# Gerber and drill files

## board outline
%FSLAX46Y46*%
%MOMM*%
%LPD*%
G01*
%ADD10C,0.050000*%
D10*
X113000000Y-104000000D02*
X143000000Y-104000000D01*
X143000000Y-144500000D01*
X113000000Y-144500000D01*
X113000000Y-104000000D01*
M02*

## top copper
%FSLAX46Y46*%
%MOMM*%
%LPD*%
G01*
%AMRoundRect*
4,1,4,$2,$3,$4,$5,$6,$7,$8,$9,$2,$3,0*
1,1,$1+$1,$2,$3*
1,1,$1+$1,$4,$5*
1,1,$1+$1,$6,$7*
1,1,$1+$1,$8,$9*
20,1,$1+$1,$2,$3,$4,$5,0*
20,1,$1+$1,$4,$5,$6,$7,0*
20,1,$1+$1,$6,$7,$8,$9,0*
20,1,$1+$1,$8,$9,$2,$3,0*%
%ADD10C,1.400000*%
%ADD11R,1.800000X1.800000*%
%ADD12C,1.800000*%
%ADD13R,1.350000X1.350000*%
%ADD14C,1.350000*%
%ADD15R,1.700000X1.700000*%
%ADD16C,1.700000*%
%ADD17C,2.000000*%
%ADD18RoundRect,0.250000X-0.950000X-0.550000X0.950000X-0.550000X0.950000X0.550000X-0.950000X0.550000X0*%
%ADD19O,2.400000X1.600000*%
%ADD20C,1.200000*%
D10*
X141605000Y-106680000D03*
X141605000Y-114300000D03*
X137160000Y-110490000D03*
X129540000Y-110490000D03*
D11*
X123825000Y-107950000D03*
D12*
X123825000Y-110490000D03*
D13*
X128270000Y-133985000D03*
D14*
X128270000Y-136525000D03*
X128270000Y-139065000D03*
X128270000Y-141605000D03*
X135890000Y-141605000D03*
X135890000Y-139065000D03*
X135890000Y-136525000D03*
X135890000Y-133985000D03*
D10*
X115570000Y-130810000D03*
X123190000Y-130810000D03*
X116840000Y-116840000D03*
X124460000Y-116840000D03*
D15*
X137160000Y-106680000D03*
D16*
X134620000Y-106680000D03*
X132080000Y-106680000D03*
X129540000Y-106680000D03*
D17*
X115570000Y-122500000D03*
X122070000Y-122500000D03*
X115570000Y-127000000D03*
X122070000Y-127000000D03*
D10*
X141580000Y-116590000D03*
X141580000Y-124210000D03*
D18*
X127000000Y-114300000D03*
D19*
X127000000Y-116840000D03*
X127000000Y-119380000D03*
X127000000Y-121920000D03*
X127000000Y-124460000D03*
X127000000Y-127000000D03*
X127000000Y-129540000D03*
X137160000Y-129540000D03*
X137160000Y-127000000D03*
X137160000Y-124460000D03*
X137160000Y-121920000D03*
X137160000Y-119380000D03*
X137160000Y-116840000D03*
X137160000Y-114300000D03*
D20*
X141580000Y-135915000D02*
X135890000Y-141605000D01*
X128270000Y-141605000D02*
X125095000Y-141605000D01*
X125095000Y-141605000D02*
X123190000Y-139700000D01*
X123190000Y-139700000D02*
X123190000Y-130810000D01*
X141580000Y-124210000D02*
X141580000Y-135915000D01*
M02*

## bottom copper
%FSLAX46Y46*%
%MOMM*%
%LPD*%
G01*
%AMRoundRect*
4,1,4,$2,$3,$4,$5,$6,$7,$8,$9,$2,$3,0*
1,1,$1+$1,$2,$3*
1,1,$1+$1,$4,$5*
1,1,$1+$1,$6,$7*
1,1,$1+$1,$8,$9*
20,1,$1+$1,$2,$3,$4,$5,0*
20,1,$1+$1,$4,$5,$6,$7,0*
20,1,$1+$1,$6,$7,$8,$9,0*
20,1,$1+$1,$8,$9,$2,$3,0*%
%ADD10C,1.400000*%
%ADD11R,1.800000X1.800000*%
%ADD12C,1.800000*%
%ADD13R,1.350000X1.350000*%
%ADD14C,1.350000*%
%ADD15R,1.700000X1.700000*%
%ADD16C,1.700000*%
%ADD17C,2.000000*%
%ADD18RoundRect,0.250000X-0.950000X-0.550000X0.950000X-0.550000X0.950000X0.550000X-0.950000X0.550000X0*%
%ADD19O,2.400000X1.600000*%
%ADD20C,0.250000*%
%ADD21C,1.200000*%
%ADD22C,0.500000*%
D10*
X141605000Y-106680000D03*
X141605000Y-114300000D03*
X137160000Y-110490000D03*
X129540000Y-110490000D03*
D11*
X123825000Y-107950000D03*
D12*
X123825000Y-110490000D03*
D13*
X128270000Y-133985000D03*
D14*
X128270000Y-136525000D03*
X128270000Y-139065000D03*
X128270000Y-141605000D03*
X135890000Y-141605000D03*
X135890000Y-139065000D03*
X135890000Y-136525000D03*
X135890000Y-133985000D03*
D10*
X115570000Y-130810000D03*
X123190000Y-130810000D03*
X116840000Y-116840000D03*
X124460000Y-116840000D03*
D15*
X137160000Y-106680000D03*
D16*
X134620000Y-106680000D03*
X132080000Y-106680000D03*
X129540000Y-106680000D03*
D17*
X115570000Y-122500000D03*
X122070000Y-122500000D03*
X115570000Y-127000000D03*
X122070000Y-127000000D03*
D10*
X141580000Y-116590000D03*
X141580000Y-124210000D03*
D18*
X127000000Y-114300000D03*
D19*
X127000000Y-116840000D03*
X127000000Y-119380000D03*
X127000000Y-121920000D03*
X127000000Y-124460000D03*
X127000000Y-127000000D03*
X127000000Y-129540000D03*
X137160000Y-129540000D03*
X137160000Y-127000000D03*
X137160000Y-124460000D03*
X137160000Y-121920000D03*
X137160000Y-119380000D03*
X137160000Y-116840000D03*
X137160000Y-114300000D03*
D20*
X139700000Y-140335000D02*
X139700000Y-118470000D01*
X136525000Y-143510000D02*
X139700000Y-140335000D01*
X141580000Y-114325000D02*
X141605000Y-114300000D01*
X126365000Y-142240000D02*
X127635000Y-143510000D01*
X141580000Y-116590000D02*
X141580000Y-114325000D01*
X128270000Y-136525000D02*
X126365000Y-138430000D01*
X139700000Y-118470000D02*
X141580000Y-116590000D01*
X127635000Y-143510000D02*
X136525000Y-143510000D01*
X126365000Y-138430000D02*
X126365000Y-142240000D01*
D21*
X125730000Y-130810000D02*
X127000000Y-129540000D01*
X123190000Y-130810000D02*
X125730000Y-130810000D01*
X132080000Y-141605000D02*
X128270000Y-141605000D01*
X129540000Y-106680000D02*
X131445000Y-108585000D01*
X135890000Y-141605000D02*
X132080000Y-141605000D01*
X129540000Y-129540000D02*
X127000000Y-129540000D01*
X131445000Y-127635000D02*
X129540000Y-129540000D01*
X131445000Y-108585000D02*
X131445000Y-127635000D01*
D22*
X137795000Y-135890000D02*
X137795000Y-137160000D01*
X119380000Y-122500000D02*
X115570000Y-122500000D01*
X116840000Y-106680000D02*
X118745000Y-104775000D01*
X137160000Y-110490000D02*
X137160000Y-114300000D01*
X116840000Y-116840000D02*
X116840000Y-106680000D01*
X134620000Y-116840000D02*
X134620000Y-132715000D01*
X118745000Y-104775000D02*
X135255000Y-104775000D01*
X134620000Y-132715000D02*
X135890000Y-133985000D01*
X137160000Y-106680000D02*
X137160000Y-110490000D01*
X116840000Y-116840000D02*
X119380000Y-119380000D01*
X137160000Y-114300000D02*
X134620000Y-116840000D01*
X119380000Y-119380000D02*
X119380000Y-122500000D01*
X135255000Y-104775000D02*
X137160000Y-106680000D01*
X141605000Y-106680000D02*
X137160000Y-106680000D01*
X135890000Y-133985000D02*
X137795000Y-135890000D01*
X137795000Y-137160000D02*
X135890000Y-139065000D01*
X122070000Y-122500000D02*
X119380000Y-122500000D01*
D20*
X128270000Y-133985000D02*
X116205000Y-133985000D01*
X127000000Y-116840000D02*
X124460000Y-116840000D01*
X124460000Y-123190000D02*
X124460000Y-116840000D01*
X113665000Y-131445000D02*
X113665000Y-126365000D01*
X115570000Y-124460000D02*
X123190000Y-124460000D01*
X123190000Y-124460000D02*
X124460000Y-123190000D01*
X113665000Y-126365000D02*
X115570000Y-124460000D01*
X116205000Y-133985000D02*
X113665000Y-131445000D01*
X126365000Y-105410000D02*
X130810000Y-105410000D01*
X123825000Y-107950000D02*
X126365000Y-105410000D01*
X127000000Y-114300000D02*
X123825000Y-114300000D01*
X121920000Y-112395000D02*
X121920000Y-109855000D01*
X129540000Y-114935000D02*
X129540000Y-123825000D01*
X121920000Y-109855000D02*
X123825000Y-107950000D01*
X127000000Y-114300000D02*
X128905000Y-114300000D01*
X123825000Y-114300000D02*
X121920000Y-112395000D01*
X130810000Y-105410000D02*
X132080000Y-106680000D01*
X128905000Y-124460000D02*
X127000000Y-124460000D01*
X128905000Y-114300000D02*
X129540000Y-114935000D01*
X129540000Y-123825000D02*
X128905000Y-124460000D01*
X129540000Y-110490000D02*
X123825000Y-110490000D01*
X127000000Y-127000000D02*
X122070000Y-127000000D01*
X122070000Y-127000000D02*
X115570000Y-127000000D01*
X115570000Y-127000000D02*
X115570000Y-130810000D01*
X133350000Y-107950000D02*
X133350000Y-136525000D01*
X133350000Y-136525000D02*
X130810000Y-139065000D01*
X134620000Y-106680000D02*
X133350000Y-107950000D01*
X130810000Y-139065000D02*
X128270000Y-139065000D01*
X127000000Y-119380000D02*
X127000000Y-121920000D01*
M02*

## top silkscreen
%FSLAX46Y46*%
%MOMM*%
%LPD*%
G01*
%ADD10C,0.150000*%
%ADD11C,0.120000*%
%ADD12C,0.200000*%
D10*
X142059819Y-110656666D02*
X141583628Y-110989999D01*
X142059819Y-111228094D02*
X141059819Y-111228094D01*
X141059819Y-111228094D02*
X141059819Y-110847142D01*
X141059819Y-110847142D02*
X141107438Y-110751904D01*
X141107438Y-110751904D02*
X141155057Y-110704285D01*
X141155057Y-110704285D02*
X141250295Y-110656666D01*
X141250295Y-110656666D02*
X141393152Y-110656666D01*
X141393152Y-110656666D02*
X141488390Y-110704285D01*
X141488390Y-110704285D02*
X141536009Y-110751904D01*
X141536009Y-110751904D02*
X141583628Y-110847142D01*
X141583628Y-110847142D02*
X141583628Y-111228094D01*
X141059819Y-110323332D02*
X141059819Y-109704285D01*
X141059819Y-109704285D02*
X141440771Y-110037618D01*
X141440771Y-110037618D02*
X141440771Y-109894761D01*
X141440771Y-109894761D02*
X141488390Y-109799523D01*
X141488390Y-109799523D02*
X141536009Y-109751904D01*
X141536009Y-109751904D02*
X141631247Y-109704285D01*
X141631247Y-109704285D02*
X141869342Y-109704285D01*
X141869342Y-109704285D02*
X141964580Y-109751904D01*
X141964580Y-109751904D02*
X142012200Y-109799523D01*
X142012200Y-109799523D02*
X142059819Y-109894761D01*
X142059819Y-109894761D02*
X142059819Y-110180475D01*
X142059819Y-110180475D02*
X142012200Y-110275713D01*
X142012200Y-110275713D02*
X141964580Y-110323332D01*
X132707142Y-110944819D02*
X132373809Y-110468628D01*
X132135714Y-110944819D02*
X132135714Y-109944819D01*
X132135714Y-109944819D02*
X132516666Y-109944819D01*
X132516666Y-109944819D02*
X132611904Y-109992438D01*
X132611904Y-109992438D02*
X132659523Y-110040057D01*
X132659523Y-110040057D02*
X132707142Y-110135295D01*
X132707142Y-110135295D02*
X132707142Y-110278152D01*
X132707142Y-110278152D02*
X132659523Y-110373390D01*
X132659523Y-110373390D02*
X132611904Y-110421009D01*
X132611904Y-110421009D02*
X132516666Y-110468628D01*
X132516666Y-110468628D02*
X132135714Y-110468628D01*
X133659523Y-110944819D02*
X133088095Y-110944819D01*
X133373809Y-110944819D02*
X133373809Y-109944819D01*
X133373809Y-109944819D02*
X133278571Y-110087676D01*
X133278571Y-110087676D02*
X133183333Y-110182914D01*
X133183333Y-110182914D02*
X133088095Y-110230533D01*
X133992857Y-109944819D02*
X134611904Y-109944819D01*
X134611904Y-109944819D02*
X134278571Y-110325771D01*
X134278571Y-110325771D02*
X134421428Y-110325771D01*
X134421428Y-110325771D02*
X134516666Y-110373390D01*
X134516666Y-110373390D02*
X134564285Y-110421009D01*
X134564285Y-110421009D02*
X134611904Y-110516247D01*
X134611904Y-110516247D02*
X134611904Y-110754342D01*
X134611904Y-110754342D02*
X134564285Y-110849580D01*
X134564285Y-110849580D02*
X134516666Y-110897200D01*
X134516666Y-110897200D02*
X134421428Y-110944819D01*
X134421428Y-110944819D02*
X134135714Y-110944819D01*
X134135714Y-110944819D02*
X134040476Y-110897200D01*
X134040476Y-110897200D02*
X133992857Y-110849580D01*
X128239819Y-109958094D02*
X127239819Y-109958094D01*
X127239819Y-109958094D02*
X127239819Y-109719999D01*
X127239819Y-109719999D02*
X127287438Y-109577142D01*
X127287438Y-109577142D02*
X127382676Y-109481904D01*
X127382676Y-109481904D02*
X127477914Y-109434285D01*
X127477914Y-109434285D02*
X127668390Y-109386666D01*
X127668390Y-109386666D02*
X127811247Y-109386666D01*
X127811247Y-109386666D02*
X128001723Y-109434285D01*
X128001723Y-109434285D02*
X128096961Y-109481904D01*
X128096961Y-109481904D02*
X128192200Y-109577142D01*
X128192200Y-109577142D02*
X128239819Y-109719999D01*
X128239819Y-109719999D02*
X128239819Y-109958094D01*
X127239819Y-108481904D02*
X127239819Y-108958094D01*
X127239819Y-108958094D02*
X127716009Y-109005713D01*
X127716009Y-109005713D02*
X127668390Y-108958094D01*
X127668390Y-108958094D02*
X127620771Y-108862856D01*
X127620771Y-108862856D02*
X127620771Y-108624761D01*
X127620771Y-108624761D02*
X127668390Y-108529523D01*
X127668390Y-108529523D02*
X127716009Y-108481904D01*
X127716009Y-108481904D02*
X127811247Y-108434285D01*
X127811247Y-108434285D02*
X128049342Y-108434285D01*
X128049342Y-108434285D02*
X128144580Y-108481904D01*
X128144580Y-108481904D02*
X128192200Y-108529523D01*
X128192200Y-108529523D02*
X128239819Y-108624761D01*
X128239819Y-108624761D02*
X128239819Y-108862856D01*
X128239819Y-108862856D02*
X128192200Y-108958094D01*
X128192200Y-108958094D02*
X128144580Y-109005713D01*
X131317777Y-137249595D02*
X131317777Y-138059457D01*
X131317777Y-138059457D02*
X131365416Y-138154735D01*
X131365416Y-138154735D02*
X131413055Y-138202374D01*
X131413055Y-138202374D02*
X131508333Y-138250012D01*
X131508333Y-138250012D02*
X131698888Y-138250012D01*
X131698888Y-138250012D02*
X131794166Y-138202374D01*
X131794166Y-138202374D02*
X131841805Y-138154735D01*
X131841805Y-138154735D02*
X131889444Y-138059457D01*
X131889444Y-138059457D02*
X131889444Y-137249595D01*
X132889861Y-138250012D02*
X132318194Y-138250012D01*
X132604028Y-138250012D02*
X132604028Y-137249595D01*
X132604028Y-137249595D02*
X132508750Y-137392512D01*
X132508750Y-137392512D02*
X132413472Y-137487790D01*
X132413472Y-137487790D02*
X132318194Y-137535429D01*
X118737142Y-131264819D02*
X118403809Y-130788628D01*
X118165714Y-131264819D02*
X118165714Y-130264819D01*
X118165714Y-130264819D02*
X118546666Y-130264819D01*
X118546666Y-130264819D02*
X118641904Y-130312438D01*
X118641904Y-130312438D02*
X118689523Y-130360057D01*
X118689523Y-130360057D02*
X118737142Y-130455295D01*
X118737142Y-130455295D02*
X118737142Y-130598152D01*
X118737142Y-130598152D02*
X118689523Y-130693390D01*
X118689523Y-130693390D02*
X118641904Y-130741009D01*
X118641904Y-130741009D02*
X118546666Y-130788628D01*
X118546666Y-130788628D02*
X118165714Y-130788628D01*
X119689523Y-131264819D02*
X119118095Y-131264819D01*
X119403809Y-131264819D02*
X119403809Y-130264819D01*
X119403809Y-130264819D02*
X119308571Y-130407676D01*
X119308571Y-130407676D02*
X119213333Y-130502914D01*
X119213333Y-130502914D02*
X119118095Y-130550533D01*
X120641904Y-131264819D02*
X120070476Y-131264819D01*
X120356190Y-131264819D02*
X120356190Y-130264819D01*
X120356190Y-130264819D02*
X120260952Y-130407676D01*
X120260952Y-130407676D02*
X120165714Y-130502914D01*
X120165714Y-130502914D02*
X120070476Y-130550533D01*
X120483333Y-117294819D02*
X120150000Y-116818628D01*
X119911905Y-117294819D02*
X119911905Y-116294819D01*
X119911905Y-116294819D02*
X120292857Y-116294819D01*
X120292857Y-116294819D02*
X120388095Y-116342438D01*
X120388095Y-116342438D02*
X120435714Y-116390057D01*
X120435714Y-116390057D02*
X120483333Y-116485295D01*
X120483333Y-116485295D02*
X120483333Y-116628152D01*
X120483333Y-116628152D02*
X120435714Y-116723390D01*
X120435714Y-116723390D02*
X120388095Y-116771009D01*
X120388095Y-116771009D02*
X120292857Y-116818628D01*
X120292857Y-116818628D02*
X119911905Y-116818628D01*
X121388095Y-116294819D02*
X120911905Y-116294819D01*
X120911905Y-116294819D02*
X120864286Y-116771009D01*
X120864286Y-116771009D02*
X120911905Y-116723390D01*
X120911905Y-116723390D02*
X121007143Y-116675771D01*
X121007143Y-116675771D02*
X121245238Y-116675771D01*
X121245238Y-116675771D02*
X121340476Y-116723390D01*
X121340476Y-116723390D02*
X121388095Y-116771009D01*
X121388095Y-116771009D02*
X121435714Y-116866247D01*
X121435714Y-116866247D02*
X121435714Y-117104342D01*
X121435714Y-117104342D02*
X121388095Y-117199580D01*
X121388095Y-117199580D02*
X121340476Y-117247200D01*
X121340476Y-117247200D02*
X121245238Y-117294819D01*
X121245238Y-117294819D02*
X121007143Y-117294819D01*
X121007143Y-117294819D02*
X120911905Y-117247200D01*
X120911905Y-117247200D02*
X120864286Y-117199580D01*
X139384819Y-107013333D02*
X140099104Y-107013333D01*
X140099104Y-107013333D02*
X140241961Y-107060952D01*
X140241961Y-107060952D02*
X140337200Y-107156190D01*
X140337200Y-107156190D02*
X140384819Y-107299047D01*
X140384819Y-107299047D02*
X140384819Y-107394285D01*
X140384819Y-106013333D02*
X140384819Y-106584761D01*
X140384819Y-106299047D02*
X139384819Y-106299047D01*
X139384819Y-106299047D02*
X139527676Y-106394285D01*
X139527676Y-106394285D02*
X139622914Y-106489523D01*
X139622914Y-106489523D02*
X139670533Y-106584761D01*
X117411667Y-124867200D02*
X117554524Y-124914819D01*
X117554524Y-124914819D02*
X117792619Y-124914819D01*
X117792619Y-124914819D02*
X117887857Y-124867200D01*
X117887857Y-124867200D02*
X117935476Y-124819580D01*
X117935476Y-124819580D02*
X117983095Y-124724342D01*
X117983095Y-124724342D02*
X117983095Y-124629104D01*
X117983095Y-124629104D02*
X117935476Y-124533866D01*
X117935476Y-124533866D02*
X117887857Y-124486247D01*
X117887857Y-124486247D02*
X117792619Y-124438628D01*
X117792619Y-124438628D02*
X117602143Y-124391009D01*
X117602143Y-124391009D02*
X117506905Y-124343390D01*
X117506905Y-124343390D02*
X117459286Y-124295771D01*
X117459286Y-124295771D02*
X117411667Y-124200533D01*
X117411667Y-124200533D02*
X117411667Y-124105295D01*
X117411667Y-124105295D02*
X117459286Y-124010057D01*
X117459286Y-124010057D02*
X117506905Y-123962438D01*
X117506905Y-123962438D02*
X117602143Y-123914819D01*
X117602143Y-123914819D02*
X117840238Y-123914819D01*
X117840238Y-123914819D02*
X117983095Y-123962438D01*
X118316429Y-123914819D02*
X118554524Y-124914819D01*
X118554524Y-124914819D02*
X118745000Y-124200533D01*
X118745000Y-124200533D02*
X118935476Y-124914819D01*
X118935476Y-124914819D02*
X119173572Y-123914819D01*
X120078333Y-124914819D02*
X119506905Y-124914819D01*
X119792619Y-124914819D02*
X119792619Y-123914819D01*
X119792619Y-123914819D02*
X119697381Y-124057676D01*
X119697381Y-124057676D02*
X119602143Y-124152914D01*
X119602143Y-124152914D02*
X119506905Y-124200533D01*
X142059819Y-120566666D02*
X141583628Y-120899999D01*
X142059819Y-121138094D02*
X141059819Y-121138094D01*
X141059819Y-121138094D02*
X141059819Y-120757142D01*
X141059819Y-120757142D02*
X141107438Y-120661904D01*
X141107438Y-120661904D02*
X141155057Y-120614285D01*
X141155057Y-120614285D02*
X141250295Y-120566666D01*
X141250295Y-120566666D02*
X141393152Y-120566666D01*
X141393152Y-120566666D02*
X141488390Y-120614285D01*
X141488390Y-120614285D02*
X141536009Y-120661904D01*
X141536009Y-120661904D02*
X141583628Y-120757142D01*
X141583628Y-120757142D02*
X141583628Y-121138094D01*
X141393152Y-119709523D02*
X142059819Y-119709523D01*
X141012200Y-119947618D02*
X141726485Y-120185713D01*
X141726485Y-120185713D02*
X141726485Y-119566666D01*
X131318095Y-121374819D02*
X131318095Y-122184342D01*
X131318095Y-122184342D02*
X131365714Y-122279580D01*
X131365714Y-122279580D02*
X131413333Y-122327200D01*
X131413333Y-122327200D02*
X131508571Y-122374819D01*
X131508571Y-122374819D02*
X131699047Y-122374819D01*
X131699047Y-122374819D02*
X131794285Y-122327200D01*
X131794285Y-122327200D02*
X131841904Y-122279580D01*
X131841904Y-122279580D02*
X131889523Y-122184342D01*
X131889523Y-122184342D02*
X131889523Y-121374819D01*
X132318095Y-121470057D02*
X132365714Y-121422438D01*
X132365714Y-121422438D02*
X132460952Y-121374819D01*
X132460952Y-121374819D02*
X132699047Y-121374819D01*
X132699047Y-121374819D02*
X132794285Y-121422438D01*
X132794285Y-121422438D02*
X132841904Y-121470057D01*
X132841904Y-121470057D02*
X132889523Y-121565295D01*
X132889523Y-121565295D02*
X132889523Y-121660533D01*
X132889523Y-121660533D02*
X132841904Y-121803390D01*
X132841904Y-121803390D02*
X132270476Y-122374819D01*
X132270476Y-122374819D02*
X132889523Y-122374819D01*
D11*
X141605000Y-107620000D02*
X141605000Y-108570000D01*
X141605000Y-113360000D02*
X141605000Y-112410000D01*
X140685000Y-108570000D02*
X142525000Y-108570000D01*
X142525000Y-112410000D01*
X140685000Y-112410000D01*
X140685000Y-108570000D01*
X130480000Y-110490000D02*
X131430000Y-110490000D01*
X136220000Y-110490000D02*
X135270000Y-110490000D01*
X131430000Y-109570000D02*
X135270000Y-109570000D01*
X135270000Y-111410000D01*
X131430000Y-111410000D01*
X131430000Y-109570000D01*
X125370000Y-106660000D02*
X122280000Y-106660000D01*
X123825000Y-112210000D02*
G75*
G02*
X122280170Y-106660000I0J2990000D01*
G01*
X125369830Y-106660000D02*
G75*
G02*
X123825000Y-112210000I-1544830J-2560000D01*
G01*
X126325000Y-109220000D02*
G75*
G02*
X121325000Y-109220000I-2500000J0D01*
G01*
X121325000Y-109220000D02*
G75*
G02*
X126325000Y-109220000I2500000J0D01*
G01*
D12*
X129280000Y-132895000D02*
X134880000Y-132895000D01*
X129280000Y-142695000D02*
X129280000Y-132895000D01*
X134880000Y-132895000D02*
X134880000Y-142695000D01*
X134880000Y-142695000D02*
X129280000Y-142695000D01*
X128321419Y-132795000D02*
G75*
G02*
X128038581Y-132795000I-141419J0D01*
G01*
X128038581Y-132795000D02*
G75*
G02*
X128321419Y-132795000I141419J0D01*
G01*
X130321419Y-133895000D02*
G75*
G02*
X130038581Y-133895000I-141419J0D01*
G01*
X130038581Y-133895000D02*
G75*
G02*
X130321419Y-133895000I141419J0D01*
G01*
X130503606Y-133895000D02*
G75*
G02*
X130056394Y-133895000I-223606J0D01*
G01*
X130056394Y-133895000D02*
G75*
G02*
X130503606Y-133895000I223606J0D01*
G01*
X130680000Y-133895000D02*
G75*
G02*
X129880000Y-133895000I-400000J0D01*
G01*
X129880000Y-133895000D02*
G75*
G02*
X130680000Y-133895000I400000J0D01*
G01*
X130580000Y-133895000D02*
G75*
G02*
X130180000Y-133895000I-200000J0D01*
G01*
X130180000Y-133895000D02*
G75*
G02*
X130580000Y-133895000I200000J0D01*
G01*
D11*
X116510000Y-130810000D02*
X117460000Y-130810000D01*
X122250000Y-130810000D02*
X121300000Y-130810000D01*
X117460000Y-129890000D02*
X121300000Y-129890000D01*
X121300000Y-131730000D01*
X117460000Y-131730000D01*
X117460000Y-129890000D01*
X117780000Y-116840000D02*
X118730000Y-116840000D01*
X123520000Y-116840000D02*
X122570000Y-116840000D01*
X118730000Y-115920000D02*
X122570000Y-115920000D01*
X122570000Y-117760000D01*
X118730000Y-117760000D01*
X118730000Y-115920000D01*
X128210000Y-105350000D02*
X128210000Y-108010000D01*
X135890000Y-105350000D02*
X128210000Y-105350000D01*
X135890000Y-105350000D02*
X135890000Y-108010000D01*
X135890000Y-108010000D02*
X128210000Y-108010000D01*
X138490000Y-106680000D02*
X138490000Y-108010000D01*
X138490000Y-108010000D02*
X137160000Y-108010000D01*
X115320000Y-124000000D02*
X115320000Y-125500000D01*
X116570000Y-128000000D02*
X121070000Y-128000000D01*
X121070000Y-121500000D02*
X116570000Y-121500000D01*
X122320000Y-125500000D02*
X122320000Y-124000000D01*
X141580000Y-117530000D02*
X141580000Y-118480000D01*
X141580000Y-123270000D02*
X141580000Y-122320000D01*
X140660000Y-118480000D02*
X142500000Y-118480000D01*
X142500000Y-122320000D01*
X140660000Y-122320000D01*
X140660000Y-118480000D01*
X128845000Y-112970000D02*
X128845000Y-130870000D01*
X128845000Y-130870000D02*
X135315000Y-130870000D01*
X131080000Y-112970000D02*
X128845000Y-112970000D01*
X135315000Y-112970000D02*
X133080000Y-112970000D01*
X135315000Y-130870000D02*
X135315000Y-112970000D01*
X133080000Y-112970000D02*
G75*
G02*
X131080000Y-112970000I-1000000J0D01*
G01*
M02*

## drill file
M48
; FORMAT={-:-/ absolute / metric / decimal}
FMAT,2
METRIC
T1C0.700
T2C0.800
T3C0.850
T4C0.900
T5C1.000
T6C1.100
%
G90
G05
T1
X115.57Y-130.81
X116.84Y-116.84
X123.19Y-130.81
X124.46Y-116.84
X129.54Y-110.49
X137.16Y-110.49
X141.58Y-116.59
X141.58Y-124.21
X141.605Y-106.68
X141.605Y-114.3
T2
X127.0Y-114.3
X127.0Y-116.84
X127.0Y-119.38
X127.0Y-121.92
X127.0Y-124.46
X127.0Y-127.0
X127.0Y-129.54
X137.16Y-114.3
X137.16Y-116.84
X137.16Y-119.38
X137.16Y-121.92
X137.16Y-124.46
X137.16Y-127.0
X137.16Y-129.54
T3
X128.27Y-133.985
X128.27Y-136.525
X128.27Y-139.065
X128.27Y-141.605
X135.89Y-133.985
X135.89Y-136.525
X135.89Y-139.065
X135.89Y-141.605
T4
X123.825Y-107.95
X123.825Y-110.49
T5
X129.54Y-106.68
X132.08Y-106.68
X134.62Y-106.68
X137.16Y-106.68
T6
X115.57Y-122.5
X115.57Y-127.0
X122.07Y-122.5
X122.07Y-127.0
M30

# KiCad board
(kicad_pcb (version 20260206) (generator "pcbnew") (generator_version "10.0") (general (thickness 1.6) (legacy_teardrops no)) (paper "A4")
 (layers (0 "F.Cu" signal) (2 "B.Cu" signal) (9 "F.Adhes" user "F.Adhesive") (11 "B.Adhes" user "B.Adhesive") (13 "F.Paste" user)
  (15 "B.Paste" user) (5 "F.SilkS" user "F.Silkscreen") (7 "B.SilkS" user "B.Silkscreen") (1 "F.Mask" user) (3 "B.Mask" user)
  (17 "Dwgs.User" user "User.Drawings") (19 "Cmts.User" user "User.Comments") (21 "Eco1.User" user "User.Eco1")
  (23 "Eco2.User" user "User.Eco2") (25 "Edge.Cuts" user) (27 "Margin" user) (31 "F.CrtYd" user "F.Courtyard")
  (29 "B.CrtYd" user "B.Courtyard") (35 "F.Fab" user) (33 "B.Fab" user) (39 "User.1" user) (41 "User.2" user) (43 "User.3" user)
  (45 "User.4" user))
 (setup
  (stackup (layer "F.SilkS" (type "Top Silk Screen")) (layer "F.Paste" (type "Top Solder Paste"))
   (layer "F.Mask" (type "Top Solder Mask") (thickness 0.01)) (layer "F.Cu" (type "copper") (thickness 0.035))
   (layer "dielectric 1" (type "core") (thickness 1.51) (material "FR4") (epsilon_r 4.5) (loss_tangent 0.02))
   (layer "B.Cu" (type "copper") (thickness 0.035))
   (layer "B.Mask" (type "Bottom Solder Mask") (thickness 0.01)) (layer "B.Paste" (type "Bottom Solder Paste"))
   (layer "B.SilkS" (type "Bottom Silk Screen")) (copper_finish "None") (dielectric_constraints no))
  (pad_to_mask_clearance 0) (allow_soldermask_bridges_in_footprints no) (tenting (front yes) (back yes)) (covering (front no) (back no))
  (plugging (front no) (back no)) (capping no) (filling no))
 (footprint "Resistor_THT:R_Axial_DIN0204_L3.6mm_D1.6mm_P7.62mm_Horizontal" (layer "F.Cu") (at 141.605 106.68 -90)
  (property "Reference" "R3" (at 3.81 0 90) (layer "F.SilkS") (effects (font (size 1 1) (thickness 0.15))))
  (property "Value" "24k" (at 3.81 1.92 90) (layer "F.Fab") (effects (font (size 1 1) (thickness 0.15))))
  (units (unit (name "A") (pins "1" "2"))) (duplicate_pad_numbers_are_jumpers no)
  (fp_line (start 0.94 0) (end 1.89 0) (stroke (width 0.12) (type solid)) (layer "F.SilkS"))
  (fp_line (start 6.68 0) (end 5.73 0) (stroke (width 0.12) (type solid)) (layer "F.SilkS"))
  (fp_rect (start 1.89 -0.92) (end 5.73 0.92) (stroke (width 0.12) (type solid)) (fill no) (layer "F.SilkS"))
  (pad "1" thru_hole circle (at 0 0 270) (size 1.4 1.4) (drill 0.7) (layers "*.Cu" "*.Mask") (remove_unused_layers no) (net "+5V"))
  (pad "2" thru_hole circle (at 7.62 0 270) (size 1.4 1.4) (drill 0.7) (layers "*.Cu" "*.Mask") (remove_unused_layers no)
   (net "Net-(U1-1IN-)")))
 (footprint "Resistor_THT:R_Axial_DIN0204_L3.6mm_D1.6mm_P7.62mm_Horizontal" (layer "F.Cu") (at 137.16 110.49 180)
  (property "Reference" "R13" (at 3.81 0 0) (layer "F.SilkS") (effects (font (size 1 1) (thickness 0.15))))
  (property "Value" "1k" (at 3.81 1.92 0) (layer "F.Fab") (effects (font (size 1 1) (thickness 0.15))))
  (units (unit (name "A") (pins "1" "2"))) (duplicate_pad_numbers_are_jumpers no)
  (fp_line (start 6.68 0) (end 5.73 0) (stroke (width 0.12) (type solid)) (layer "F.SilkS"))
  (fp_line (start 0.94 0) (end 1.89 0) (stroke (width 0.12) (type solid)) (layer "F.SilkS"))
  (fp_rect (start 1.89 -0.92) (end 5.73 0.92) (stroke (width 0.12) (type solid)) (fill no) (layer "F.SilkS"))
  (pad "1" thru_hole circle (at 0 0 180) (size 1.4 1.4) (drill 0.7) (layers "*.Cu" "*.Mask") (remove_unused_layers no) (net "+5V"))
  (pad "2" thru_hole circle (at 7.62 0 180) (size 1.4 1.4) (drill 0.7) (layers "*.Cu" "*.Mask") (remove_unused_layers no) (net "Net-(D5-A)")))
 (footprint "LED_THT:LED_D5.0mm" (layer "F.Cu") (at 123.825 107.95 -90)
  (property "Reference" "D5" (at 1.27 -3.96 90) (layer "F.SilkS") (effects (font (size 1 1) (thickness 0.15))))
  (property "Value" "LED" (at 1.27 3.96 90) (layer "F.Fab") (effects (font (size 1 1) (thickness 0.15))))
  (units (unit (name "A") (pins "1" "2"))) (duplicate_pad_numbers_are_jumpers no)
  (fp_line (start -1.29 -1.545) (end -1.29 1.545) (stroke (width 0.12) (type solid)) (layer "F.SilkS"))
  (fp_arc (start 4.26 0) (mid 2.071779 2.880495) (end -1.29 1.54483) (stroke (width 0.12) (type solid)) (layer "F.SilkS"))
  (fp_arc (start -1.29 -1.54483) (mid 2.071779 -2.880495) (end 4.26 0) (stroke (width 0.12) (type solid)) (layer "F.SilkS"))
  (fp_circle (center 1.27 0) (end 3.77 0) (stroke (width 0.12) (type solid)) (fill no) (layer "F.SilkS"))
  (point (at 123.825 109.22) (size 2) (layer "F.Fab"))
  (pad "1" thru_hole rect (at 0 0 270) (size 1.8 1.8) (drill 0.9) (layers "*.Cu" "*.Mask") (remove_unused_layers no) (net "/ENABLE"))
  (pad "2" thru_hole circle (at 2.54 0 270) (size 1.8 1.8) (drill 0.9) (layers "*.Cu" "*.Mask") (remove_unused_layers no) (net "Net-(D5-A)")))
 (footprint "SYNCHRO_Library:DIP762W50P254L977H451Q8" (layer "F.Cu") (at 132.08 137.795)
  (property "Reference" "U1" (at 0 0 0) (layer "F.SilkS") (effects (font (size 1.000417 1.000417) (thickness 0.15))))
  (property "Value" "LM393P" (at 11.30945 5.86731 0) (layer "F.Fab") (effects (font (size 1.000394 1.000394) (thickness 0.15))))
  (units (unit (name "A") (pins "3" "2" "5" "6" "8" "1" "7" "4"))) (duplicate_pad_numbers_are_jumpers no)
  (fp_line (start -2.8 -4.9) (end 2.8 -4.9) (stroke (width 0.2) (type solid)) (layer "F.SilkS"))
  (fp_line (start -2.8 4.9) (end -2.8 -4.9) (stroke (width 0.2) (type solid)) (layer "F.SilkS"))
  (fp_line (start 2.8 -4.9) (end 2.8 4.9) (stroke (width 0.2) (type solid)) (layer "F.SilkS"))
  (fp_line (start 2.8 4.9) (end -2.8 4.9) (stroke (width 0.2) (type solid)) (layer "F.SilkS"))
  (fp_circle (center -3.9 -5) (end -3.758581 -5) (stroke (width 0.2) (type solid)) (fill no) (layer "F.SilkS"))
  (fp_circle (center -1.9 -3.9) (end -1.758581 -3.9) (stroke (width 0.2) (type solid)) (fill no) (layer "F.SilkS"))
  (fp_circle (center -1.8 -3.9) (end -1.576394 -3.9) (stroke (width 0.2) (type solid)) (fill no) (layer "F.SilkS"))
  (fp_circle (center -1.8 -3.9) (end -1.4 -3.9) (stroke (width 0.2) (type solid)) (fill no) (layer "F.SilkS"))
  (fp_circle (center -1.7 -3.9) (end -1.5 -3.9) (stroke (width 0.2) (type solid)) (fill no) (layer "F.SilkS"))
  (pad "1" thru_hole rect (at -3.81 -3.81) (size 1.35 1.35) (drill 0.85) (layers "*.Cu" "*.Mask") (remove_unused_layers no)
   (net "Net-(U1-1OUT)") (solder_mask_margin 0.102))
  (pad "2" thru_hole circle (at -3.81 -1.27) (size 1.35 1.35) (drill 0.85) (layers "*.Cu" "*.Mask") (remove_unused_layers no)
   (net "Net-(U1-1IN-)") (solder_mask_margin 0.102))
  (pad "3" thru_hole circle (at -3.81 1.27) (size 1.35 1.35) (drill 0.85) (layers "*.Cu" "*.Mask") (remove_unused_layers no) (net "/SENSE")
   (solder_mask_margin 0.102))
  (pad "4" thru_hole circle (at -3.81 3.81) (size 1.35 1.35) (drill 0.85) (layers "*.Cu" "*.Mask") (remove_unused_layers no) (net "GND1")
   (solder_mask_margin 0.102))
  (pad "5" thru_hole circle (at 3.81 3.81) (size 1.35 1.35) (drill 0.85) (layers "*.Cu" "*.Mask") (remove_unused_layers no) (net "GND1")
   (solder_mask_margin 0.102))
  (pad "6" thru_hole circle (at 3.81 1.27) (size 1.35 1.35) (drill 0.85) (layers "*.Cu" "*.Mask") (remove_unused_layers no) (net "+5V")
   (solder_mask_margin 0.102))
  (pad "7" thru_hole circle (at 3.81 -1.27) (size 1.35 1.35) (drill 0.85) (layers "*.Cu" "*.Mask") (remove_unused_layers no)
   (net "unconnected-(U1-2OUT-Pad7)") (solder_mask_margin 0.102))
  (pad "8" thru_hole circle (at 3.81 -3.81) (size 1.35 1.35) (drill 0.85) (layers "*.Cu" "*.Mask") (remove_unused_layers no) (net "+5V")
   (solder_mask_margin 0.102)))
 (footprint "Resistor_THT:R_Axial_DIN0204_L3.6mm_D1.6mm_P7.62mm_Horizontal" (layer "F.Cu") (at 115.57 130.81)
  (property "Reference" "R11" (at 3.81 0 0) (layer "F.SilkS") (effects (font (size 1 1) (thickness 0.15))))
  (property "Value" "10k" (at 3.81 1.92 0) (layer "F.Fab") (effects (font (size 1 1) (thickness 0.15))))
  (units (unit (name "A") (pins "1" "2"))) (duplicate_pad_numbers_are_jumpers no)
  (fp_line (start 0.94 0) (end 1.89 0) (stroke (width 0.12) (type solid)) (layer "F.SilkS"))
  (fp_line (start 6.68 0) (end 5.73 0) (stroke (width 0.12) (type solid)) (layer "F.SilkS"))
  (fp_rect (start 1.89 -0.92) (end 5.73 0.92) (stroke (width 0.12) (type solid)) (fill no) (layer "F.SilkS"))
  (pad "1" thru_hole circle (at 0 0) (size 1.4 1.4) (drill 0.7) (layers "*.Cu" "*.Mask") (remove_unused_layers no) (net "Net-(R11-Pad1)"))
  (pad "2" thru_hole circle (at 7.62 0) (size 1.4 1.4) (drill 0.7) (layers "*.Cu" "*.Mask") (remove_unused_layers no) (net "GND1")))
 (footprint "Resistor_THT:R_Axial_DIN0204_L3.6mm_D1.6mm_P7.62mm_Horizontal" (layer "F.Cu") (at 116.84 116.84)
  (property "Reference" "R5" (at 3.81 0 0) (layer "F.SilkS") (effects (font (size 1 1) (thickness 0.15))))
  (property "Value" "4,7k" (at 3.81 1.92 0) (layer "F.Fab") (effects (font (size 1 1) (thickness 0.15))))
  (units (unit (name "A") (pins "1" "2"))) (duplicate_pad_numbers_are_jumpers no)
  (fp_line (start 0.94 0) (end 1.89 0) (stroke (width 0.12) (type solid)) (layer "F.SilkS"))
  (fp_line (start 6.68 0) (end 5.73 0) (stroke (width 0.12) (type solid)) (layer "F.SilkS"))
  (fp_rect (start 1.89 -0.92) (end 5.73 0.92) (stroke (width 0.12) (type solid)) (fill no) (layer "F.SilkS"))
  (pad "1" thru_hole circle (at 0 0) (size 1.4 1.4) (drill 0.7) (layers "*.Cu" "*.Mask") (remove_unused_layers no) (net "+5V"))
  (pad "2" thru_hole circle (at 7.62 0) (size 1.4 1.4) (drill 0.7) (layers "*.Cu" "*.Mask") (remove_unused_layers no) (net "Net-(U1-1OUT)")))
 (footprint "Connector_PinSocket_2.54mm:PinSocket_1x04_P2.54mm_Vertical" (layer "F.Cu") (at 137.16 106.68 -90)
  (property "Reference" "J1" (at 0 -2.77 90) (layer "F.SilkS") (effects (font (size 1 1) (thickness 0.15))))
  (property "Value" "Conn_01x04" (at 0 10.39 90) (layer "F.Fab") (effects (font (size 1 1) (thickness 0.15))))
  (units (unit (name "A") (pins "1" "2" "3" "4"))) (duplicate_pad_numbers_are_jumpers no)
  (fp_line (start -1.33 8.95) (end 1.33 8.95) (stroke (width 0.12) (type solid)) (layer "F.SilkS"))
  (fp_line (start -1.33 1.27) (end -1.33 8.95) (stroke (width 0.12) (type solid)) (layer "F.SilkS"))
  (fp_line (start -1.33 1.27) (end 1.33 1.27) (stroke (width 0.12) (type solid)) (layer "F.SilkS"))
  (fp_line (start 1.33 1.27) (end 1.33 8.95) (stroke (width 0.12) (type solid)) (layer "F.SilkS"))
  (fp_line (start 0 -1.33) (end 1.33 -1.33) (stroke (width 0.12) (type solid)) (layer "F.SilkS"))
  (fp_line (start 1.33 -1.33) (end 1.33 0) (stroke (width 0.12) (type solid)) (layer "F.SilkS"))
  (pad "1" thru_hole rect (at 0 0 270) (size 1.7 1.7) (drill 1) (layers "*.Cu" "*.Mask") (remove_unused_layers no) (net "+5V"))
  (pad "2" thru_hole circle (at 0 2.54 270) (size 1.7 1.7) (drill 1) (layers "*.Cu" "*.Mask") (remove_unused_layers no) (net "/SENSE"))
  (pad "3" thru_hole circle (at 0 5.08 270) (size 1.7 1.7) (drill 1) (layers "*.Cu" "*.Mask") (remove_unused_layers no) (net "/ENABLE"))
  (pad "4" thru_hole circle (at 0 7.62 270) (size 1.7 1.7) (drill 1) (layers "*.Cu" "*.Mask") (remove_unused_layers no) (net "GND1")))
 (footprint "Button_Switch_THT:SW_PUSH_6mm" (layer "F.Cu") (at 115.57 122.5)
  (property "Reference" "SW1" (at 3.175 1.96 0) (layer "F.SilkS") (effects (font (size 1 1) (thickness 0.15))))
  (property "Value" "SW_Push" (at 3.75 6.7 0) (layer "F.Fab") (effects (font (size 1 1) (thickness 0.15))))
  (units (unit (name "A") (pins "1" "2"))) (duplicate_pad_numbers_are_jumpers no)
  (fp_line (start -0.25 1.5) (end -0.25 3) (stroke (width 0.12) (type solid)) (layer "F.SilkS"))
  (fp_line (start 1 5.5) (end 5.5 5.5) (stroke (width 0.12) (type solid)) (layer "F.SilkS"))
  (fp_line (start 5.5 -1) (end 1 -1) (stroke (width 0.12) (type solid)) (layer "F.SilkS"))
  (fp_line (start 6.75 3) (end 6.75 1.5) (stroke (width 0.12) (type solid)) (layer "F.SilkS"))
  (pad "1" thru_hole circle (at 0 0 90) (size 2 2) (drill 1.1) (layers "*.Cu" "*.Mask") (remove_unused_layers no) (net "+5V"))
  (pad "1" thru_hole circle (at 6.5 0 90) (size 2 2) (drill 1.1) (layers "*.Cu" "*.Mask") (remove_unused_layers no) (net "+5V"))
  (pad "2" thru_hole circle (at 0 4.5 90) (size 2 2) (drill 1.1) (layers "*.Cu" "*.Mask") (remove_unused_layers no) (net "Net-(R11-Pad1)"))
  (pad "2" thru_hole circle (at 6.5 4.5 90) (size 2 2) (drill 1.1) (layers "*.Cu" "*.Mask") (remove_unused_layers no) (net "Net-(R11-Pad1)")))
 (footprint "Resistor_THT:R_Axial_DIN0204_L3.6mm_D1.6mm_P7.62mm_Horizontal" (layer "F.Cu") (at 141.58 116.59 -90)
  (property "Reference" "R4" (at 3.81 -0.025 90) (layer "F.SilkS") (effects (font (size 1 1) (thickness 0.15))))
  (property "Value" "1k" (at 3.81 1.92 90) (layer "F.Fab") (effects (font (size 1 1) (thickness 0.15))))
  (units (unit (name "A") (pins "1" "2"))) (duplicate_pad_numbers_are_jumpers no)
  (fp_line (start 0.94 0) (end 1.89 0) (stroke (width 0.12) (type solid)) (layer "F.SilkS"))
  (fp_line (start 6.68 0) (end 5.73 0) (stroke (width 0.12) (type solid)) (layer "F.SilkS"))
  (fp_rect (start 1.89 -0.92) (end 5.73 0.92) (stroke (width 0.12) (type solid)) (fill no) (layer "F.SilkS"))
  (pad "1" thru_hole circle (at 0 0 270) (size 1.4 1.4) (drill 0.7) (layers "*.Cu" "*.Mask") (remove_unused_layers no) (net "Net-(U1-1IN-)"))
  (pad "2" thru_hole circle (at 7.62 0 270) (size 1.4 1.4) (drill 0.7) (layers "*.Cu" "*.Mask") (remove_unused_layers no) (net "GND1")))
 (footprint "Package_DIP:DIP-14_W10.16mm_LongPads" (layer "F.Cu") (at 127 114.3)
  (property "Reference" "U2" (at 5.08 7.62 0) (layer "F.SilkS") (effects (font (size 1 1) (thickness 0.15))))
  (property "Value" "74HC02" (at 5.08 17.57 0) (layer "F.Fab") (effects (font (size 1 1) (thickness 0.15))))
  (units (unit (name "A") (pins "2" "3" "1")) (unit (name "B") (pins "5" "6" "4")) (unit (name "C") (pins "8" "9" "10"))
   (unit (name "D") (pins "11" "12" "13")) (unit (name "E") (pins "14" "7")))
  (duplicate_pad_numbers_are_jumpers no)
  (fp_line (start 1.845 -1.33) (end 1.845 16.57) (stroke (width 0.12) (type solid)) (layer "F.SilkS"))
  (fp_line (start 1.845 16.57) (end 8.315 16.57) (stroke (width 0.12) (type solid)) (layer "F.SilkS"))
  (fp_line (start 4.08 -1.33) (end 1.845 -1.33) (stroke (width 0.12) (type solid)) (layer "F.SilkS"))
  (fp_line (start 8.315 -1.33) (end 6.08 -1.33) (stroke (width 0.12) (type solid)) (layer "F.SilkS"))
  (fp_line (start 8.315 16.57) (end 8.315 -1.33) (stroke (width 0.12) (type solid)) (layer "F.SilkS"))
  (fp_arc (start 6.08 -1.33) (mid 5.08 -0.33) (end 4.08 -1.33) (stroke (width 0.12) (type solid)) (layer "F.SilkS"))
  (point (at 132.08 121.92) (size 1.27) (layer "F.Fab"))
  (pad "1" thru_hole roundrect (at 0 0) (size 2.4 1.6) (drill 0.8) (layers "*.Cu" "*.Mask") (remove_unused_layers no)
   (roundrect_rratio 0.15625) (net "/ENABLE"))
  (pad "2" thru_hole oval (at 0 2.54) (size 2.4 1.6) (drill 0.8) (layers "*.Cu" "*.Mask") (remove_unused_layers no) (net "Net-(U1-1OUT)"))
  (pad "3" thru_hole oval (at 0 5.08) (size 2.4 1.6) (drill 0.8) (layers "*.Cu" "*.Mask") (remove_unused_layers no) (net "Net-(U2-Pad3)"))
  (pad "4" thru_hole oval (at 0 7.62) (size 2.4 1.6) (drill 0.8) (layers "*.Cu" "*.Mask") (remove_unused_layers no) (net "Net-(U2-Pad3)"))
  (pad "5" thru_hole oval (at 0 10.16) (size 2.4 1.6) (drill 0.8) (layers "*.Cu" "*.Mask") (remove_unused_layers no) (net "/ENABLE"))
  (pad "6" thru_hole oval (at 0 12.7) (size 2.4 1.6) (drill 0.8) (layers "*.Cu" "*.Mask") (remove_unused_layers no) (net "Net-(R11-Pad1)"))
  (pad "7" thru_hole oval (at 0 15.24) (size 2.4 1.6) (drill 0.8) (layers "*.Cu" "*.Mask") (remove_unused_layers no) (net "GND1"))
  (pad "8" thru_hole oval (at 10.16 15.24) (size 2.4 1.6) (drill 0.8) (layers "*.Cu" "*.Mask") (remove_unused_layers no))
  (pad "9" thru_hole oval (at 10.16 12.7) (size 2.4 1.6) (drill 0.8) (layers "*.Cu" "*.Mask") (remove_unused_layers no))
  (pad "10" thru_hole oval (at 10.16 10.16) (size 2.4 1.6) (drill 0.8) (layers "*.Cu" "*.Mask") (remove_unused_layers no))
  (pad "11" thru_hole oval (at 10.16 7.62) (size 2.4 1.6) (drill 0.8) (layers "*.Cu" "*.Mask") (remove_unused_layers no))
  (pad "12" thru_hole oval (at 10.16 5.08) (size 2.4 1.6) (drill 0.8) (layers "*.Cu" "*.Mask") (remove_unused_layers no))
  (pad "13" thru_hole oval (at 10.16 2.54) (size 2.4 1.6) (drill 0.8) (layers "*.Cu" "*.Mask") (remove_unused_layers no))
  (pad "14" thru_hole oval (at 10.16 0) (size 2.4 1.6) (drill 0.8) (layers "*.Cu" "*.Mask") (remove_unused_layers no) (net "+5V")))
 (gr_rect (start 113 104) (end 143 144.5) (stroke (width 0.05) (type default)) (fill no) (layer "Edge.Cuts"))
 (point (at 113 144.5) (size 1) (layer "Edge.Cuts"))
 (segment (start 139.7 140.335) (end 139.7 118.47) (width 0.25) (layer "B.Cu") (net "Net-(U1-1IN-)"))
 (segment (start 136.525 143.51) (end 139.7 140.335) (width 0.25) (layer "B.Cu") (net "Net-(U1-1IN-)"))
 (segment (start 141.58 114.325) (end 141.605 114.3) (width 0.25) (layer "B.Cu") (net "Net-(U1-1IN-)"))
 (segment (start 126.365 142.24) (end 127.635 143.51) (width 0.25) (layer "B.Cu") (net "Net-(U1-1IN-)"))
 (segment (start 141.58 116.59) (end 141.58 114.325) (width 0.25) (layer "B.Cu") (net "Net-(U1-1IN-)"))
 (segment (start 128.27 136.525) (end 126.365 138.43) (width 0.25) (layer "B.Cu") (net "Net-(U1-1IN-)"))
 (segment (start 139.7 118.47) (end 141.58 116.59) (width 0.25) (layer "B.Cu") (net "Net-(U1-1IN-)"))
 (segment (start 127.635 143.51) (end 136.525 143.51) (width 0.25) (layer "B.Cu") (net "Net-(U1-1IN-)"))
 (segment (start 126.365 138.43) (end 126.365 142.24) (width 0.25) (layer "B.Cu") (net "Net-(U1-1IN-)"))
 (segment (start 141.58 135.915) (end 135.89 141.605) (width 1.2) (layer "F.Cu") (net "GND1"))
 (segment (start 128.27 141.605) (end 125.095 141.605) (width 1.2) (layer "F.Cu") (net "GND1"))
 (segment (start 125.095 141.605) (end 123.19 139.7) (width 1.2) (layer "F.Cu") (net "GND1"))
 (segment (start 123.19 139.7) (end 123.19 130.81) (width 1.2) (layer "F.Cu") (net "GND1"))
 (segment (start 141.58 124.21) (end 141.58 135.915) (width 1.2) (layer "F.Cu") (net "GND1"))
 (segment (start 125.73 130.81) (end 127 129.54) (width 1.2) (layer "B.Cu") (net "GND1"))
 (segment (start 123.19 130.81) (end 125.73 130.81) (width 1.2) (layer "B.Cu") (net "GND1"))
 (segment (start 132.08 141.605) (end 128.27 141.605) (width 1.2) (layer "B.Cu") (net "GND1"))
 (segment (start 129.54 106.68) (end 131.445 108.585) (width 1.2) (layer "B.Cu") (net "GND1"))
 (segment (start 135.89 141.605) (end 132.08 141.605) (width 1.2) (layer "B.Cu") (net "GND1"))
 (segment (start 129.54 129.54) (end 127 129.54) (width 1.2) (layer "B.Cu") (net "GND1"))
 (segment (start 131.445 127.635) (end 129.54 129.54) (width 1.2) (layer "B.Cu") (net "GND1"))
 (segment (start 131.445 108.585) (end 131.445 127.635) (width 1.2) (layer "B.Cu") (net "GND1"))
 (segment (start 137.795 135.89) (end 137.795 137.16) (width 0.5) (layer "B.Cu") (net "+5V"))
 (segment (start 119.38 122.5) (end 115.57 122.5) (width 0.5) (layer "B.Cu") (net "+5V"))
 (segment (start 116.84 106.68) (end 118.745 104.775) (width 0.5) (layer "B.Cu") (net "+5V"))
 (segment (start 137.16 110.49) (end 137.16 114.3) (width 0.5) (layer "B.Cu") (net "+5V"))
 (segment (start 116.84 116.84) (end 116.84 106.68) (width 0.5) (layer "B.Cu") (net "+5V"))
 (segment (start 134.62 116.84) (end 134.62 132.715) (width 0.5) (layer "B.Cu") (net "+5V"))
 (segment (start 118.745 104.775) (end 135.255 104.775) (width 0.5) (layer "B.Cu") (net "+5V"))
 (segment (start 134.62 132.715) (end 135.89 133.985) (width 0.5) (layer "B.Cu") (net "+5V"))
 (segment (start 137.16 106.68) (end 137.16 110.49) (width 0.5) (layer "B.Cu") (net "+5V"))
 (segment (start 116.84 116.84) (end 119.38 119.38) (width 0.5) (layer "B.Cu") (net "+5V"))
 (segment (start 137.16 114.3) (end 134.62 116.84) (width 0.5) (layer "B.Cu") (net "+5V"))
 (segment (start 119.38 119.38) (end 119.38 122.5) (width 0.5) (layer "B.Cu") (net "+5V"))
 (segment (start 135.255 104.775) (end 137.16 106.68) (width 0.5) (layer "B.Cu") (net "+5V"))
 (segment (start 141.605 106.68) (end 137.16 106.68) (width 0.5) (layer "B.Cu") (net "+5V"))
 (segment (start 135.89 133.985) (end 137.795 135.89) (width 0.5) (layer "B.Cu") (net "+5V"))
 (segment (start 137.795 137.16) (end 135.89 139.065) (width 0.5) (layer "B.Cu") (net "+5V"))
 (segment (start 122.07 122.5) (end 119.38 122.5) (width 0.5) (layer "B.Cu") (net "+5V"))
 (segment (start 128.27 133.985) (end 116.205 133.985) (width 0.25) (layer "B.Cu") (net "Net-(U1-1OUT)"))
 (segment (start 127 116.84) (end 124.46 116.84) (width 0.25) (layer "B.Cu") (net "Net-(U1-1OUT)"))
 (segment (start 124.46 123.19) (end 124.46 116.84) (width 0.25) (layer "B.Cu") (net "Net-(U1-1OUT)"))
 (segment (start 113.665 131.445) (end 113.665 126.365) (width 0.25) (layer "B.Cu") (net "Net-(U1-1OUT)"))
 (segment (start 115.57 124.46) (end 123.19 124.46) (width 0.25) (layer "B.Cu") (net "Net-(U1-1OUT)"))
 (segment (start 123.19 124.46) (end 124.46 123.19) (width 0.25) (layer "B.Cu") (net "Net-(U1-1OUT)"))
 (segment (start 113.665 126.365) (end 115.57 124.46) (width 0.25) (layer "B.Cu") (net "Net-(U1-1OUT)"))
 (segment (start 116.205 133.985) (end 113.665 131.445) (width 0.25) (layer "B.Cu") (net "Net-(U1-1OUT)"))
 (segment (start 126.365 105.41) (end 130.81 105.41) (width 0.25) (layer "B.Cu") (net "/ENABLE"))
 (segment (start 123.825 107.95) (end 126.365 105.41) (width 0.25) (layer "B.Cu") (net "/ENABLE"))
 (segment (start 127 114.3) (end 123.825 114.3) (width 0.25) (layer "B.Cu") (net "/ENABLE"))
 (segment (start 121.92 112.395) (end 121.92 109.855) (width 0.25) (layer "B.Cu") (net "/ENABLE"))
 (segment (start 129.54 114.935) (end 129.54 123.825) (width 0.25) (layer "B.Cu") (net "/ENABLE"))
 (segment (start 121.92 109.855) (end 123.825 107.95) (width 0.25) (layer "B.Cu") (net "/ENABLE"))
 (segment (start 127 114.3) (end 128.905 114.3) (width 0.25) (layer "B.Cu") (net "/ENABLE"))
 (segment (start 123.825 114.3) (end 121.92 112.395) (width 0.25) (layer "B.Cu") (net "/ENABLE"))
 (segment (start 130.81 105.41) (end 132.08 106.68) (width 0.25) (layer "B.Cu") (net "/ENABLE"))
 (segment (start 128.905 124.46) (end 127 124.46) (width 0.25) (layer "B.Cu") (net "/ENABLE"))
 (segment (start 128.905 114.3) (end 129.54 114.935) (width 0.25) (layer "B.Cu") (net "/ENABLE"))
 (segment (start 129.54 123.825) (end 128.905 124.46) (width 0.25) (layer "B.Cu") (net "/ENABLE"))
 (segment (start 129.54 110.49) (end 123.825 110.49) (width 0.25) (layer "B.Cu") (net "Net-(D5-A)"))
 (segment (start 127 127) (end 122.07 127) (width 0.25) (layer "B.Cu") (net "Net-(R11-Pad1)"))
 (segment (start 122.07 127) (end 115.57 127) (width 0.25) (layer "B.Cu") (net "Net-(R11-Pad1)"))
 (segment (start 115.57 127) (end 115.57 130.81) (width 0.25) (layer "B.Cu") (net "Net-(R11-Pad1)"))
 (segment (start 133.35 107.95) (end 133.35 136.525) (width 0.25) (layer "B.Cu") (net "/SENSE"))
 (segment (start 133.35 136.525) (end 130.81 139.065) (width 0.25) (layer "B.Cu") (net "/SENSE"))
 (segment (start 134.62 106.68) (end 133.35 107.95) (width 0.25) (layer "B.Cu") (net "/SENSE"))
 (segment (start 130.81 139.065) (end 128.27 139.065) (width 0.25) (layer "B.Cu") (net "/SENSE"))
 (segment (start 127 119.38) (end 127 121.92) (width 0.25) (layer "B.Cu") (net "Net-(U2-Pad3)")))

